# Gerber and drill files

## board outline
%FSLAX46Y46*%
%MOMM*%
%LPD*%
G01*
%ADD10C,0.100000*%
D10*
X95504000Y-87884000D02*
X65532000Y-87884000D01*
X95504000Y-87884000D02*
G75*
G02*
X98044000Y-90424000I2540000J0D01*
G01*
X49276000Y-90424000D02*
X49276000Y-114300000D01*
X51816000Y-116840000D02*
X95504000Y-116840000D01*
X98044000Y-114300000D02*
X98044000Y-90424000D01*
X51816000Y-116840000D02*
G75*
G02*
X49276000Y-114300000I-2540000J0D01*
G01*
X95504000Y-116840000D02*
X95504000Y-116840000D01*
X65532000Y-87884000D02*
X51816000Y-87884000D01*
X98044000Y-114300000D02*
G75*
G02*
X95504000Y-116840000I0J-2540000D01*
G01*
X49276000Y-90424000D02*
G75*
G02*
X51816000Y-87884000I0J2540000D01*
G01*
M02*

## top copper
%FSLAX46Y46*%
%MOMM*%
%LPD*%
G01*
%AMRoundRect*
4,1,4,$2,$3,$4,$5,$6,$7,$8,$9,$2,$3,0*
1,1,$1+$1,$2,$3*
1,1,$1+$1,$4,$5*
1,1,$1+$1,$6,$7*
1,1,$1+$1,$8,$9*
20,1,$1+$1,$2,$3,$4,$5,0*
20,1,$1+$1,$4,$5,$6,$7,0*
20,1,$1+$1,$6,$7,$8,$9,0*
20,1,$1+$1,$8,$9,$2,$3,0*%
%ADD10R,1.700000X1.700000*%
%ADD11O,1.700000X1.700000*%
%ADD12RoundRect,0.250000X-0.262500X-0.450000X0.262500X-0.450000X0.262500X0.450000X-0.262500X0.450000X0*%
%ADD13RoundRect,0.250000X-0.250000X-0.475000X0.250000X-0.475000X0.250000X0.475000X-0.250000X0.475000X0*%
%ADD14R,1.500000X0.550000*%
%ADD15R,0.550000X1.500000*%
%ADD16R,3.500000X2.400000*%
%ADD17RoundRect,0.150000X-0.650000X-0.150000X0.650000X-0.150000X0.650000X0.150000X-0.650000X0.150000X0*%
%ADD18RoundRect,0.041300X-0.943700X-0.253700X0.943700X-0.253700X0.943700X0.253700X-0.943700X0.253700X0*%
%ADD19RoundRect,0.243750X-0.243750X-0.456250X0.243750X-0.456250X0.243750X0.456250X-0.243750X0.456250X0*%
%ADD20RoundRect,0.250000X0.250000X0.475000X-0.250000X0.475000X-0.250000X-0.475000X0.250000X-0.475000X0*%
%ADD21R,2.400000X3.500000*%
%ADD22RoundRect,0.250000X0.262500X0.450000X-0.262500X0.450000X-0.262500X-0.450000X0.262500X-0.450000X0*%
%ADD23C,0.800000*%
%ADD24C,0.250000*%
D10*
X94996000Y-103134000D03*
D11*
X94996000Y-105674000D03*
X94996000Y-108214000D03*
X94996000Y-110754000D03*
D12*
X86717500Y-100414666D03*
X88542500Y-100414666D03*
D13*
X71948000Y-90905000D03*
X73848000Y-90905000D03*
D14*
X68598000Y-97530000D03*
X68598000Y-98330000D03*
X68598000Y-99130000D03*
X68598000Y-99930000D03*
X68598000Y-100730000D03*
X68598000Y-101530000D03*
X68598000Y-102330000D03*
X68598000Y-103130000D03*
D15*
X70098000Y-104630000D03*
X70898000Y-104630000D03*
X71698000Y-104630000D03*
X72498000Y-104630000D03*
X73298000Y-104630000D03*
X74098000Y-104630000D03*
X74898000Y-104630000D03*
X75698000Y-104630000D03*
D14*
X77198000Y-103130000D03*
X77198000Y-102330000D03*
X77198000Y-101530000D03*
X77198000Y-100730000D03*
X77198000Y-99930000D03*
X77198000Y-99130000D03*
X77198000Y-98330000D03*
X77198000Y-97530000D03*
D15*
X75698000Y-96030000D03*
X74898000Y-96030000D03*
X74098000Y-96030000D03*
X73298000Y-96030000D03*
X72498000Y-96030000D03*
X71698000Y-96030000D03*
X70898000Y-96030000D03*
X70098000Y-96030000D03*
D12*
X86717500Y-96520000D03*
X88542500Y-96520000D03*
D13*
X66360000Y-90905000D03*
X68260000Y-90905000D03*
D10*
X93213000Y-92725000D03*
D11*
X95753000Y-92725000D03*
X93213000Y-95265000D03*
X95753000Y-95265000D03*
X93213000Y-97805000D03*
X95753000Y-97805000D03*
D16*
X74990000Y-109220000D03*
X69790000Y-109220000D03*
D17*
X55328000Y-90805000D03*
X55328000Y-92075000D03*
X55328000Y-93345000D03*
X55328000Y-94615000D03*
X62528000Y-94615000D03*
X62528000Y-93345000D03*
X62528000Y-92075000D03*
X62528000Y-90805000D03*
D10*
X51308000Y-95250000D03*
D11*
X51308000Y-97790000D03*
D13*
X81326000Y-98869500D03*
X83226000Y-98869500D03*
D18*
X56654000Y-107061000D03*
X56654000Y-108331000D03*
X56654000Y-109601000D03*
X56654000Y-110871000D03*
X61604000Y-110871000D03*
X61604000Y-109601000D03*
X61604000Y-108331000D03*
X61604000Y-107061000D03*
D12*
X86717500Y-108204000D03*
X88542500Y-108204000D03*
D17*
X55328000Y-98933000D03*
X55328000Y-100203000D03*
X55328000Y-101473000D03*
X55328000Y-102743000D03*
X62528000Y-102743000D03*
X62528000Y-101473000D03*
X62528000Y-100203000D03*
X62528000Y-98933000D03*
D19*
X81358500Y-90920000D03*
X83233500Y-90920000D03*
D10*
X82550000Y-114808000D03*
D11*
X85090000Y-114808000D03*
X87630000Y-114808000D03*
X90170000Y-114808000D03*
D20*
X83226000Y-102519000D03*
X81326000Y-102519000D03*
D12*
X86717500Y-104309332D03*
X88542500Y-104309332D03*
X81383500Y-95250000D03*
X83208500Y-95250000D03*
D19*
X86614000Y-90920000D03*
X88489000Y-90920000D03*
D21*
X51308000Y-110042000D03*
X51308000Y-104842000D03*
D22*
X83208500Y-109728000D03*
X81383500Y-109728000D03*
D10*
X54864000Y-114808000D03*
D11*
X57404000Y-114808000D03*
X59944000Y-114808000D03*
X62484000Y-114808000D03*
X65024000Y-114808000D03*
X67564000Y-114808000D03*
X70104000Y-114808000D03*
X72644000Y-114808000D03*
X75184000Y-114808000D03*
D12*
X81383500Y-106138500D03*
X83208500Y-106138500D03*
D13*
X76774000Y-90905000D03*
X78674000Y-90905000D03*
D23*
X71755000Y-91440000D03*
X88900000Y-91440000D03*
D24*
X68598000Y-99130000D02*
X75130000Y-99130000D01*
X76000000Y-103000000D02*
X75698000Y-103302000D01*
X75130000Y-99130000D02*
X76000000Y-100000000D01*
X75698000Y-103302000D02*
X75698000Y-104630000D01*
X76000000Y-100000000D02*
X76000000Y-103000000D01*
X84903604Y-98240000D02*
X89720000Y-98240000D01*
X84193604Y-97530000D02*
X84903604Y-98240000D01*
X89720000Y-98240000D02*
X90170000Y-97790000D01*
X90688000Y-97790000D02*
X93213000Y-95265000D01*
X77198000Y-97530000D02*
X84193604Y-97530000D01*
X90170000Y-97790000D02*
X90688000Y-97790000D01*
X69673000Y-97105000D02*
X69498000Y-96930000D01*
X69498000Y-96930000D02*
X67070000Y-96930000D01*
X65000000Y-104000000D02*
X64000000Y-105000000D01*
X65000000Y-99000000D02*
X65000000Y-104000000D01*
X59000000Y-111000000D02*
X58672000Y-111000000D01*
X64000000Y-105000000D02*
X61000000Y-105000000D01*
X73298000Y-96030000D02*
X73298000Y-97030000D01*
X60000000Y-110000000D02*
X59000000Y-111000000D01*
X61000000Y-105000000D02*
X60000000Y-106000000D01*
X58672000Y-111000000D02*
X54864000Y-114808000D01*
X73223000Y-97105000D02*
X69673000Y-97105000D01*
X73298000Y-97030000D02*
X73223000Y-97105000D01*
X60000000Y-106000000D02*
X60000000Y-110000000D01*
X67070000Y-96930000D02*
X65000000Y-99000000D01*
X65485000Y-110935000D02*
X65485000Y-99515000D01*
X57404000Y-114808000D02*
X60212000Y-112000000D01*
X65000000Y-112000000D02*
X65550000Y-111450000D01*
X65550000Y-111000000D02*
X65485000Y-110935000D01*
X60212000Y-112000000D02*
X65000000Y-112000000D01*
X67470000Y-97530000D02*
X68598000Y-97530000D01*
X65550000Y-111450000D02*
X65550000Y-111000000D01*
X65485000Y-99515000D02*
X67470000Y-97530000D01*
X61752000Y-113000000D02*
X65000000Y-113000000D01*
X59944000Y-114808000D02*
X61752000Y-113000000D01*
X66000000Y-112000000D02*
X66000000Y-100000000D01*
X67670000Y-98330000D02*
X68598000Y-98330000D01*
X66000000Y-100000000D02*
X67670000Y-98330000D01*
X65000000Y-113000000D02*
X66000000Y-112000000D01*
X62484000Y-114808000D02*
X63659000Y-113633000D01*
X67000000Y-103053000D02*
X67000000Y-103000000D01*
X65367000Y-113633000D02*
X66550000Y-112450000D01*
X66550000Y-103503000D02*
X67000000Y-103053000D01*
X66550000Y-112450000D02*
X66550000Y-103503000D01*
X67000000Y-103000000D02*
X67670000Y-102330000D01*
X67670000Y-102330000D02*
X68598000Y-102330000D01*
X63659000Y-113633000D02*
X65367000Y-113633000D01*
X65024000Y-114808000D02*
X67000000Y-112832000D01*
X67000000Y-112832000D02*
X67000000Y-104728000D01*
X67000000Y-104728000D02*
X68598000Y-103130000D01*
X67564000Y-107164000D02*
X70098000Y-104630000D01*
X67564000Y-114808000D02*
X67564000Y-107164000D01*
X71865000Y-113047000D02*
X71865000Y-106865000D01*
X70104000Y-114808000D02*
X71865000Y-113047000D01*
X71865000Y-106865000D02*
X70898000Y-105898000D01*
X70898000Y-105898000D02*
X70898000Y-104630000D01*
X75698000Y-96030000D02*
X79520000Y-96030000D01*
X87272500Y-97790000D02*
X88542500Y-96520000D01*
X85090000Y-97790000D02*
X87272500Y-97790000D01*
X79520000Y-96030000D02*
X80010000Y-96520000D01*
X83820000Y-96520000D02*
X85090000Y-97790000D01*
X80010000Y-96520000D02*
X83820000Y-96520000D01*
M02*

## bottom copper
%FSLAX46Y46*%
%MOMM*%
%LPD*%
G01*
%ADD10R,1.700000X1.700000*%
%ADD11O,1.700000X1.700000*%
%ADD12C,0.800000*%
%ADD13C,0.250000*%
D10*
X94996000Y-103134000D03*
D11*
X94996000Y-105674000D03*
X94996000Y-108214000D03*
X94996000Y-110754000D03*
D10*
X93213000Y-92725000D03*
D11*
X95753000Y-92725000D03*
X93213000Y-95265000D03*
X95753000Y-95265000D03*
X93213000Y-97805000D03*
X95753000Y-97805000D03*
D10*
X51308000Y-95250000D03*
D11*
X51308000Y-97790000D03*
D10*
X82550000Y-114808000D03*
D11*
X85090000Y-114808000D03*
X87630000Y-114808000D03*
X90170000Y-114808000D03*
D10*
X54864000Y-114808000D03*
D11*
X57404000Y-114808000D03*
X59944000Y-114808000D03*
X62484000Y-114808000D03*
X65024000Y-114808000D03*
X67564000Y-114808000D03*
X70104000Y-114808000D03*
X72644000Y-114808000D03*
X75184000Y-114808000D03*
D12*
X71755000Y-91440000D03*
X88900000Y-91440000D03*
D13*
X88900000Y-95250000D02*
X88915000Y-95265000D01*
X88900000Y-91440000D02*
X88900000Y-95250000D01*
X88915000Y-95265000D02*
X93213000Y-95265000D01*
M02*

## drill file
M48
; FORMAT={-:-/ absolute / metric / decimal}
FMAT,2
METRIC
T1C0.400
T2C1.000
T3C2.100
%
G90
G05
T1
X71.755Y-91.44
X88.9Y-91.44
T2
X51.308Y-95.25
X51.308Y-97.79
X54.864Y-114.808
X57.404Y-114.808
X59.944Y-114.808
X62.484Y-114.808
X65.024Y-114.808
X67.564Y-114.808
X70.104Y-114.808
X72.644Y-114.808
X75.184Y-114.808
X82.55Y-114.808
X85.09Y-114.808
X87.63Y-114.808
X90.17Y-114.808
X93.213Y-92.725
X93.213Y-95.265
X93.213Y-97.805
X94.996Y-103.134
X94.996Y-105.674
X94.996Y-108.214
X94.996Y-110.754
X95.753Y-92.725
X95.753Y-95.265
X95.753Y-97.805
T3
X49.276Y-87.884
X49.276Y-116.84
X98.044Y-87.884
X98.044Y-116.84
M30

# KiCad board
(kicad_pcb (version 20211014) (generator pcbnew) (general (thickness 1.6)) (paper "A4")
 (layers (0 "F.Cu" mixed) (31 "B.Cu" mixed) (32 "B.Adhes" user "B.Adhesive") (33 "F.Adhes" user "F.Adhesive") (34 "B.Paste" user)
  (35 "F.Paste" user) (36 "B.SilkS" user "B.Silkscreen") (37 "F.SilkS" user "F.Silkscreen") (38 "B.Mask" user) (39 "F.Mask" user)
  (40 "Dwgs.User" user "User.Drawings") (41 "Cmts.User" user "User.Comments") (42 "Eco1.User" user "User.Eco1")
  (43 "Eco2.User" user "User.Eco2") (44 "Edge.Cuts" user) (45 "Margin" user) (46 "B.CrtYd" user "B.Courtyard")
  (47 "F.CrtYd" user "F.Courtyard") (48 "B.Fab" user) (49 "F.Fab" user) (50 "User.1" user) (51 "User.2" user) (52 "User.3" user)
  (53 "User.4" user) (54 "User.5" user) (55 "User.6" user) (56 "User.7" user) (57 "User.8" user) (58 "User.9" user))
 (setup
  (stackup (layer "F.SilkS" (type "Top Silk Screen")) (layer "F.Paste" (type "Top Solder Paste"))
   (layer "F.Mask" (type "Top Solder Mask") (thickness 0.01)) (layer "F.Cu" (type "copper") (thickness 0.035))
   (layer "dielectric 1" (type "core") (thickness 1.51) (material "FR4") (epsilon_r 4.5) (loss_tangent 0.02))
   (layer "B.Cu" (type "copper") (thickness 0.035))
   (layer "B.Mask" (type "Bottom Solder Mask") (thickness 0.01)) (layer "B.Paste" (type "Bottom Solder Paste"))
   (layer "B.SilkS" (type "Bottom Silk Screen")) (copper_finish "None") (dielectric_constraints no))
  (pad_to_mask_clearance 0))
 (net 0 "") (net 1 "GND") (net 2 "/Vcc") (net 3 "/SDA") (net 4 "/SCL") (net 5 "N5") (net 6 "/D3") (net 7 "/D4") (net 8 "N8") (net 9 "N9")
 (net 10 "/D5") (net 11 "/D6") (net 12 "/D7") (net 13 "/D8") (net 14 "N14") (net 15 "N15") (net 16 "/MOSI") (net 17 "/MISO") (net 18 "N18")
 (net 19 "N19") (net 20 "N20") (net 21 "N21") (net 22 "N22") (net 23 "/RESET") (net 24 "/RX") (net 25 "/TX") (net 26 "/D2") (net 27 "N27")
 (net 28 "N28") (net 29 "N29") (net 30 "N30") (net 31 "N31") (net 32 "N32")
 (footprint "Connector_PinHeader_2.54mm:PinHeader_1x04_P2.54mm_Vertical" (layer "F.Cu") (at 94.996 103.134)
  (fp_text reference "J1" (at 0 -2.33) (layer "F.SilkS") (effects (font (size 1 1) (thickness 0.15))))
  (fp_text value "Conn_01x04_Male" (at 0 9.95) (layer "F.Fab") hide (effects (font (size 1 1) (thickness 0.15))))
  (pad "1" thru_hole rect (at 0 0) (size 1.7 1.7) (drill 1) (layers *.Cu *.Mask) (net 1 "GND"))
  (pad "2" thru_hole oval (at 0 2.54) (size 1.7 1.7) (drill 1) (layers *.Cu *.Mask) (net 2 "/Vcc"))
  (pad "3" thru_hole oval (at 0 5.08) (size 1.7 1.7) (drill 1) (layers *.Cu *.Mask) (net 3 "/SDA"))
  (pad "4" thru_hole oval (at 0 7.62) (size 1.7 1.7) (drill 1) (layers *.Cu *.Mask) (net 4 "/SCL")))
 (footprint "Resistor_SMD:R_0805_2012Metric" (layer "F.Cu") (at 87.63 100.414666)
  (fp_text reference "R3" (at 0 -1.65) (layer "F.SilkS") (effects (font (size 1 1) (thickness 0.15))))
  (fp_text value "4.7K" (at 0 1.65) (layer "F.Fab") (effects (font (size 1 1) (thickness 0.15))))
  (pad "1" smd roundrect (at -0.9125 0) (size 1.025 1.4) (layers "F.Cu" "F.Paste" "F.Mask") (roundrect_rratio 0.243902) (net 2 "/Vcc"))
  (pad "2" smd roundrect (at 0.9125 0) (size 1.025 1.4) (layers "F.Cu" "F.Paste" "F.Mask") (roundrect_rratio 0.243902) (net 3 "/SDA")))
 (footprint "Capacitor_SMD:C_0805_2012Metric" (layer "F.Cu") (at 72.898 90.905)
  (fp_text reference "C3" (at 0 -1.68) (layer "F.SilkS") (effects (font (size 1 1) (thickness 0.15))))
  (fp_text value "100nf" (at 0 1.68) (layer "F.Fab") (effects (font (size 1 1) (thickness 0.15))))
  (pad "1" smd roundrect (at -0.95 0) (size 1 1.45) (layers "F.Cu" "F.Paste" "F.Mask") (roundrect_rratio 0.25) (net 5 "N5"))
  (pad "2" smd roundrect (at 0.95 0) (size 1 1.45) (layers "F.Cu" "F.Paste" "F.Mask") (roundrect_rratio 0.25) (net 1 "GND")))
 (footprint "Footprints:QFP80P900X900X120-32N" (layer "F.Cu") (at 72.898 100.33)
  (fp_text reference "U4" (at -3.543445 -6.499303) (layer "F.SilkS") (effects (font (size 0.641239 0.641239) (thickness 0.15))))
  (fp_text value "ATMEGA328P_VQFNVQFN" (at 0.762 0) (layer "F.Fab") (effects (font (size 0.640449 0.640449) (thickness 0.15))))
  (pad "1" smd rect locked (at -4.3 -2.8) (size 1.5 0.55) (layers "F.Cu" "F.Paste" "F.Mask") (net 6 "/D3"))
  (pad "2" smd rect locked (at -4.3 -2) (size 1.5 0.55) (layers "F.Cu" "F.Paste" "F.Mask") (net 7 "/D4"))
  (pad "3" smd rect locked (at -4.3 -1.2) (size 1.5 0.55) (layers "F.Cu" "F.Paste" "F.Mask") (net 5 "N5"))
  (pad "4" smd rect locked (at -4.3 -0.4) (size 1.5 0.55) (layers "F.Cu" "F.Paste" "F.Mask") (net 1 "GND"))
  (pad "5" smd rect locked (at -4.3 0.4) (size 1.5 0.55) (layers "F.Cu" "F.Paste" "F.Mask") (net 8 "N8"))
  (pad "6" smd rect locked (at -4.3 1.2) (size 1.5 0.55) (layers "F.Cu" "F.Paste" "F.Mask") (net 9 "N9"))
  (pad "7" smd rect locked (at -4.3 2) (size 1.5 0.55) (layers "F.Cu" "F.Paste" "F.Mask") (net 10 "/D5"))
  (pad "8" smd rect locked (at -4.3 2.8) (size 1.5 0.55) (layers "F.Cu" "F.Paste" "F.Mask") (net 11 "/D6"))
  (pad "9" smd rect locked (at -2.8 4.3) (size 0.55 1.5) (layers "F.Cu" "F.Paste" "F.Mask") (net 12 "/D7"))
  (pad "10" smd rect locked (at -2 4.3) (size 0.55 1.5) (layers "F.Cu" "F.Paste" "F.Mask") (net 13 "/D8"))
  (pad "11" smd rect locked (at -1.2 4.3) (size 0.55 1.5) (layers "F.Cu" "F.Paste" "F.Mask") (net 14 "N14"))
  (pad "12" smd rect locked (at -0.4 4.3) (size 0.55 1.5) (layers "F.Cu" "F.Paste" "F.Mask") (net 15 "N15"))
  (pad "13" smd rect locked (at 0.4 4.3) (size 0.55 1.5) (layers "F.Cu" "F.Paste" "F.Mask") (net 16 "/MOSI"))
  (pad "14" smd rect locked (at 1.2 4.3) (size 0.55 1.5) (layers "F.Cu" "F.Paste" "F.Mask") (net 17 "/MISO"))
  (pad "15" smd rect locked (at 2 4.3) (size 0.55 1.5) (layers "F.Cu" "F.Paste" "F.Mask") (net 4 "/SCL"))
  (pad "16" smd rect locked (at 2.8 4.3) (size 0.55 1.5) (layers "F.Cu" "F.Paste" "F.Mask") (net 5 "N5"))
  (pad "17" smd rect locked (at 4.3 2.8) (size 1.5 0.55) (layers "F.Cu" "F.Paste" "F.Mask") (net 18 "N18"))
  (pad "18" smd rect locked (at 4.3 2) (size 1.5 0.55) (layers "F.Cu" "F.Paste" "F.Mask") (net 1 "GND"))
  (pad "19" smd rect locked (at 4.3 1.2) (size 1.5 0.55) (layers "F.Cu" "F.Paste" "F.Mask") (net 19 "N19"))
  (pad "20" smd rect locked (at 4.3 0.4) (size 1.5 0.55) (layers "F.Cu" "F.Paste" "F.Mask") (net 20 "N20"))
  (pad "21" smd rect locked (at 4.3 -0.4) (size 1.5 0.55) (layers "F.Cu" "F.Paste" "F.Mask") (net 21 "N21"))
  (pad "22" smd rect locked (at 4.3 -1.2) (size 1.5 0.55) (layers "F.Cu" "F.Paste" "F.Mask") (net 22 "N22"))
  (pad "23" smd rect locked (at 4.3 -2) (size 1.5 0.55) (layers "F.Cu" "F.Paste" "F.Mask") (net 3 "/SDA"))
  (pad "24" smd rect locked (at 4.3 -2.8) (size 1.5 0.55) (layers "F.Cu" "F.Paste" "F.Mask") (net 4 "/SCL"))
  (pad "25" smd rect locked (at 2.8 -4.3) (size 0.55 1.5) (layers "F.Cu" "F.Paste" "F.Mask") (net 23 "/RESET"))
  (pad "26" smd rect locked (at 2 -4.3) (size 0.55 1.5) (layers "F.Cu" "F.Paste" "F.Mask") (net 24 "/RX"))
  (pad "27" smd rect locked (at 1.2 -4.3) (size 0.55 1.5) (layers "F.Cu" "F.Paste" "F.Mask") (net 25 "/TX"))
  (pad "28" smd rect locked (at 0.4 -4.3) (size 0.55 1.5) (layers "F.Cu" "F.Paste" "F.Mask") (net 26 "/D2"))
  (pad "29" smd rect locked (at -0.4 -4.3) (size 0.55 1.5) (layers "F.Cu" "F.Paste" "F.Mask"))
  (pad "30" smd rect locked (at -1.2 -4.3) (size 0.55 1.5) (layers "F.Cu" "F.Paste" "F.Mask"))
  (pad "31" smd rect locked (at -2 -4.3) (size 0.55 1.5) (layers "F.Cu" "F.Paste" "F.Mask"))
  (pad "32" smd rect locked (at -2.8 -4.3) (size 0.55 1.5) (layers "F.Cu" "F.Paste" "F.Mask")))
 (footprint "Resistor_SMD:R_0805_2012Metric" (layer "F.Cu") (at 87.63 96.52)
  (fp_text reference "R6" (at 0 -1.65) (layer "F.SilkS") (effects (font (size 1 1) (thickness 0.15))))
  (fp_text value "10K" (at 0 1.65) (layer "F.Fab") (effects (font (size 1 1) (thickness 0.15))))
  (pad "1" smd roundrect (at -0.9125 0) (size 1.025 1.4) (layers "F.Cu" "F.Paste" "F.Mask") (roundrect_rratio 0.243902) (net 2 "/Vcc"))
  (pad "2" smd roundrect (at 0.9125 0) (size 1.025 1.4) (layers "F.Cu" "F.Paste" "F.Mask") (roundrect_rratio 0.243902) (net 23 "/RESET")))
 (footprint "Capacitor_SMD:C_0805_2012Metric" (layer "F.Cu") (at 67.31 90.905)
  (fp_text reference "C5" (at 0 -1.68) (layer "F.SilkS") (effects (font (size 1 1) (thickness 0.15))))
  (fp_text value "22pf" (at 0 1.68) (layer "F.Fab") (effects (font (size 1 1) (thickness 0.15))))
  (pad "1" smd roundrect (at -0.95 0) (size 1 1.45) (layers "F.Cu" "F.Paste" "F.Mask") (roundrect_rratio 0.25) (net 1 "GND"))
  (pad "2" smd roundrect (at 0.95 0) (size 1 1.45) (layers "F.Cu" "F.Paste" "F.Mask") (roundrect_rratio 0.25) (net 8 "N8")))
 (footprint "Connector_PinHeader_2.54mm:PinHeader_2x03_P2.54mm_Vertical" (layer "F.Cu") (at 93.213 92.725)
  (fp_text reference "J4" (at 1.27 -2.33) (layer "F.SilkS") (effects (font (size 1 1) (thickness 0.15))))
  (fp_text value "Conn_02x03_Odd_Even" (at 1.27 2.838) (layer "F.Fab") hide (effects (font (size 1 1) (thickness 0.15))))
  (pad "1" thru_hole rect (at 0 0) (size 1.7 1.7) (drill 1) (layers *.Cu *.Mask) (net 17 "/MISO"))
  (pad "2" thru_hole oval (at 2.54 0) (size 1.7 1.7) (drill 1) (layers *.Cu *.Mask) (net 2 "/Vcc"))
  (pad "3" thru_hole oval (at 0 2.54) (size 1.7 1.7) (drill 1) (layers *.Cu *.Mask) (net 4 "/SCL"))
  (pad "4" thru_hole oval (at 2.54 2.54) (size 1.7 1.7) (drill 1) (layers *.Cu *.Mask) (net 16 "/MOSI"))
  (pad "5" thru_hole oval (at 0 5.08) (size 1.7 1.7) (drill 1) (layers *.Cu *.Mask) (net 23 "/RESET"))
  (pad "6" thru_hole oval (at 2.54 5.08) (size 1.7 1.7) (drill 1) (layers *.Cu *.Mask) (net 1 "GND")))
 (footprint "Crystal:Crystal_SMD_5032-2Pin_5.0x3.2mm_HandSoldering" (layer "F.Cu") (at 72.39 109.22 180)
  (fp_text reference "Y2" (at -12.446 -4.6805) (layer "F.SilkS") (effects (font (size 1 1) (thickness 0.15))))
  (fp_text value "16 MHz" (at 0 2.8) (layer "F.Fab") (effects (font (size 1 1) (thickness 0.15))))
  (pad "1" smd rect (at -2.6 0 180) (size 3.5 2.4) (layers "F.Cu" "F.Paste" "F.Mask") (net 9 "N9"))
  (pad "2" smd rect (at 2.6 0 180) (size 3.5 2.4) (layers "F.Cu" "F.Paste" "F.Mask") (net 8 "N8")))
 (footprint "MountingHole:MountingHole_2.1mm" (layer "F.Cu") (at 49.276 116.84)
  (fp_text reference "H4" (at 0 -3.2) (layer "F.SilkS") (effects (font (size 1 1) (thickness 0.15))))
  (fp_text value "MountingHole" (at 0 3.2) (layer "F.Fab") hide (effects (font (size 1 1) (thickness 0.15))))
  (pad "" np_thru_hole circle (at 0 0) (size 2.1 2.1) (drill 2.1) (layers *.Cu *.Mask)))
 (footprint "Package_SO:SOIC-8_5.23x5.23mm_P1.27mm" (layer "F.Cu") (at 58.928 92.71)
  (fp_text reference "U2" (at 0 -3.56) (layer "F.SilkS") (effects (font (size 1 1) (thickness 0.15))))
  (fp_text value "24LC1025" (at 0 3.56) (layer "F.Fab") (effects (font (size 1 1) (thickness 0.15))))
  (pad "1" smd roundrect (at -3.6 -1.905) (size 1.6 0.6) (layers "F.Cu" "F.Paste" "F.Mask") (roundrect_rratio 0.25) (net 2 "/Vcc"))
  (pad "2" smd roundrect (at -3.6 -0.635) (size 1.6 0.6) (layers "F.Cu" "F.Paste" "F.Mask") (roundrect_rratio 0.25) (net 1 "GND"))
  (pad "3" smd roundrect (at -3.6 0.635) (size 1.6 0.6) (layers "F.Cu" "F.Paste" "F.Mask") (roundrect_rratio 0.25) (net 2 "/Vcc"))
  (pad "4" smd roundrect (at -3.6 1.905) (size 1.6 0.6) (layers "F.Cu" "F.Paste" "F.Mask") (roundrect_rratio 0.25) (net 1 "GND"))
  (pad "5" smd roundrect (at 3.6 1.905) (size 1.6 0.6) (layers "F.Cu" "F.Paste" "F.Mask") (roundrect_rratio 0.25) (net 3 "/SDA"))
  (pad "6" smd roundrect (at 3.6 0.635) (size 1.6 0.6) (layers "F.Cu" "F.Paste" "F.Mask") (roundrect_rratio 0.25) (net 4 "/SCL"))
  (pad "7" smd roundrect (at 3.6 -0.635) (size 1.6 0.6) (layers "F.Cu" "F.Paste" "F.Mask") (roundrect_rratio 0.25) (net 1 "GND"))
  (pad "8" smd roundrect (at 3.6 -1.905) (size 1.6 0.6) (layers "F.Cu" "F.Paste" "F.Mask") (roundrect_rratio 0.25) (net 2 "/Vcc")))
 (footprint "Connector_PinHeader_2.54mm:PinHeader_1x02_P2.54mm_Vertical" (layer "F.Cu") (at 51.308 95.25)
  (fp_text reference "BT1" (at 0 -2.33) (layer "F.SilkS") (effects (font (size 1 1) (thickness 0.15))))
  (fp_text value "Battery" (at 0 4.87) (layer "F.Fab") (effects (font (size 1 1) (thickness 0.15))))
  (pad "1" thru_hole rect (at 0 0) (size 1.7 1.7) (drill 1) (layers *.Cu *.Mask) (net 5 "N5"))
  (pad "2" thru_hole oval (at 0 2.54) (size 1.7 1.7) (drill 1) (layers *.Cu *.Mask) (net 1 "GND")))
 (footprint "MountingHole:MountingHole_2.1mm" (layer "F.Cu") (at 98.044 87.884)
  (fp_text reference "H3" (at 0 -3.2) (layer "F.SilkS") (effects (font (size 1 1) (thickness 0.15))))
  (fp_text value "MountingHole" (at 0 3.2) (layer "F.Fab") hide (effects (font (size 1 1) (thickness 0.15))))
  (pad "" np_thru_hole circle (at 0 0) (size 2.1 2.1) (drill 2.1) (layers *.Cu *.Mask)))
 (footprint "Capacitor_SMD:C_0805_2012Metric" (layer "F.Cu") (at 82.276 98.8695)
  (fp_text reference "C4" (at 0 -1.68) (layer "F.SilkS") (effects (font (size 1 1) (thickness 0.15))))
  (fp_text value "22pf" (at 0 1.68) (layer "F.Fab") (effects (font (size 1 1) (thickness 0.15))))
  (pad "1" smd roundrect (at -0.95 0) (size 1 1.45) (layers "F.Cu" "F.Paste" "F.Mask") (roundrect_rratio 0.25) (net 1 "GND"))
  (pad "2" smd roundrect (at 0.95 0) (size 1 1.45) (layers "F.Cu" "F.Paste" "F.Mask") (roundrect_rratio 0.25) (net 9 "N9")))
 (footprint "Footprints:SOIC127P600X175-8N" (layer "F.Cu") (at 59.129 108.966)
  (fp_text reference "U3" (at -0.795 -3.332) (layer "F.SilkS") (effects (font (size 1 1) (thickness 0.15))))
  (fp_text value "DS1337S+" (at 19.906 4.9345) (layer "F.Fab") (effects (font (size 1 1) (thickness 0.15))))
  (pad "1" smd roundrect locked (at -2.475 -1.905) (size 1.97 0.59) (layers "F.Cu" "F.Paste" "F.Mask") (roundrect_rratio 0.07)
   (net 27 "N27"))
  (pad "2" smd roundrect locked (at -2.475 -0.635) (size 1.97 0.59) (layers "F.Cu" "F.Paste" "F.Mask") (roundrect_rratio 0.07)
   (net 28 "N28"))
  (pad "3" smd roundrect locked (at -2.475 0.635) (size 1.97 0.59) (layers "F.Cu" "F.Paste" "F.Mask") (roundrect_rratio 0.07) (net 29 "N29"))
  (pad "4" smd roundrect locked (at -2.475 1.905) (size 1.97 0.59) (layers "F.Cu" "F.Paste" "F.Mask") (roundrect_rratio 0.07) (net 1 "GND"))
  (pad "5" smd roundrect locked (at 2.475 1.905) (size 1.97 0.59) (layers "F.Cu" "F.Paste" "F.Mask") (roundrect_rratio 0.07) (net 3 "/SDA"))
  (pad "6" smd roundrect locked (at 2.475 0.635) (size 1.97 0.59) (layers "F.Cu" "F.Paste" "F.Mask") (roundrect_rratio 0.07) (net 4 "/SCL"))
  (pad "7" smd roundrect locked (at 2.475 -0.635) (size 1.97 0.59) (layers "F.Cu" "F.Paste" "F.Mask") (roundrect_rratio 0.07) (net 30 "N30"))
  (pad "8" smd roundrect locked (at 2.475 -1.905) (size 1.97 0.59) (layers "F.Cu" "F.Paste" "F.Mask") (roundrect_rratio 0.07) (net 2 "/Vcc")))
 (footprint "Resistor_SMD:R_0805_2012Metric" (layer "F.Cu") (at 87.63 108.204)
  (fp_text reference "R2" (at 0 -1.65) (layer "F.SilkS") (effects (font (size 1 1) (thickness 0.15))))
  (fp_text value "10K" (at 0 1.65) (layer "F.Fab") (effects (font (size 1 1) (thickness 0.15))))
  (pad "1" smd roundrect (at -0.9125 0) (size 1.025 1.4) (layers "F.Cu" "F.Paste" "F.Mask") (roundrect_rratio 0.243902) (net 2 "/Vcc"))
  (pad "2" smd roundrect (at 0.9125 0) (size 1.025 1.4) (layers "F.Cu" "F.Paste" "F.Mask") (roundrect_rratio 0.243902) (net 29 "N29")))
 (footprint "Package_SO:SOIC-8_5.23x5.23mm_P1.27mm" (layer "F.Cu") (at 58.928 100.838)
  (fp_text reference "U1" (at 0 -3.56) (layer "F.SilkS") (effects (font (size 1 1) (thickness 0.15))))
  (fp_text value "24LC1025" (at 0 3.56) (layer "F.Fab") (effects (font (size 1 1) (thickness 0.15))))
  (pad "1" smd roundrect (at -3.6 -1.905) (size 1.6 0.6) (layers "F.Cu" "F.Paste" "F.Mask") (roundrect_rratio 0.25) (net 2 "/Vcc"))
  (pad "2" smd roundrect (at -3.6 -0.635) (size 1.6 0.6) (layers "F.Cu" "F.Paste" "F.Mask") (roundrect_rratio 0.25) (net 2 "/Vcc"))
  (pad "3" smd roundrect (at -3.6 0.635) (size 1.6 0.6) (layers "F.Cu" "F.Paste" "F.Mask") (roundrect_rratio 0.25) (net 2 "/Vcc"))
  (pad "4" smd roundrect (at -3.6 1.905) (size 1.6 0.6) (layers "F.Cu" "F.Paste" "F.Mask") (roundrect_rratio 0.25) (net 1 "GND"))
  (pad "5" smd roundrect (at 3.6 1.905) (size 1.6 0.6) (layers "F.Cu" "F.Paste" "F.Mask") (roundrect_rratio 0.25) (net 3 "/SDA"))
  (pad "6" smd roundrect (at 3.6 0.635) (size 1.6 0.6) (layers "F.Cu" "F.Paste" "F.Mask") (roundrect_rratio 0.25) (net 4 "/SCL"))
  (pad "7" smd roundrect (at 3.6 -0.635) (size 1.6 0.6) (layers "F.Cu" "F.Paste" "F.Mask") (roundrect_rratio 0.25) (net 1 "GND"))
  (pad "8" smd roundrect (at 3.6 -1.905) (size 1.6 0.6) (layers "F.Cu" "F.Paste" "F.Mask") (roundrect_rratio 0.25) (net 2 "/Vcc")))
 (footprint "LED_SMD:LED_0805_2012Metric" (layer "F.Cu") (at 82.296 90.92)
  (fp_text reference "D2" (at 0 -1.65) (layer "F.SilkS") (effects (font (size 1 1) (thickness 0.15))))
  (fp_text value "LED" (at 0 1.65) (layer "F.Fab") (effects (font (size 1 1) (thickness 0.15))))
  (pad "1" smd roundrect (at -0.9375 0) (size 0.975 1.4) (layers "F.Cu" "F.Paste" "F.Mask") (roundrect_rratio 0.25) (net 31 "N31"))
  (pad "2" smd roundrect (at 0.9375 0) (size 0.975 1.4) (layers "F.Cu" "F.Paste" "F.Mask") (roundrect_rratio 0.25) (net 5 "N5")))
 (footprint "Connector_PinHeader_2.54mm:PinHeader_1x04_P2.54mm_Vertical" (layer "F.Cu") (at 82.55 114.808 90)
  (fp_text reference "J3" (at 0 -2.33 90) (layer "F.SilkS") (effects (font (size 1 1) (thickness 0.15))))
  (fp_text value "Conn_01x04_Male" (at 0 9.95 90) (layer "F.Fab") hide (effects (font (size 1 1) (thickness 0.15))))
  (pad "1" thru_hole rect (at 0 0 90) (size 1.7 1.7) (drill 1) (layers *.Cu *.Mask) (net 1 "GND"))
  (pad "2" thru_hole oval (at 0 2.54 90) (size 1.7 1.7) (drill 1) (layers *.Cu *.Mask) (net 2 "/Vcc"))
  (pad "3" thru_hole oval (at 0 5.08 90) (size 1.7 1.7) (drill 1) (layers *.Cu *.Mask) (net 24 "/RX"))
  (pad "4" thru_hole oval (at 0 7.62 90) (size 1.7 1.7) (drill 1) (layers *.Cu *.Mask) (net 25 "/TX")))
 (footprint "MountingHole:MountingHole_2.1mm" (layer "F.Cu") (at 49.276 87.884)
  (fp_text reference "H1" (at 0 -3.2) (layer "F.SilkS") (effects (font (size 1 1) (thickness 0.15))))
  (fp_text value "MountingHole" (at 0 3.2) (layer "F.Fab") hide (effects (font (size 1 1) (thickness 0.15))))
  (pad "" np_thru_hole circle (at 0 0) (size 2.1 2.1) (drill 2.1) (layers *.Cu *.Mask)))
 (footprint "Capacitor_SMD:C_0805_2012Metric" (layer "F.Cu") (at 82.276 102.519 180)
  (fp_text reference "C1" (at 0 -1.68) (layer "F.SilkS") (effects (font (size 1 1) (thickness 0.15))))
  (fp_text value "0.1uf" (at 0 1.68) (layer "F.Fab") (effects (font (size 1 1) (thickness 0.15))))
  (pad "1" smd roundrect (at -0.95 0 180) (size 1 1.45) (layers "F.Cu" "F.Paste" "F.Mask") (roundrect_rratio 0.25) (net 2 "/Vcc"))
  (pad "2" smd roundrect (at 0.95 0 180) (size 1 1.45) (layers "F.Cu" "F.Paste" "F.Mask") (roundrect_rratio 0.25) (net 1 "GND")))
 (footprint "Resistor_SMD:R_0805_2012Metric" (layer "F.Cu") (at 87.63 104.309332)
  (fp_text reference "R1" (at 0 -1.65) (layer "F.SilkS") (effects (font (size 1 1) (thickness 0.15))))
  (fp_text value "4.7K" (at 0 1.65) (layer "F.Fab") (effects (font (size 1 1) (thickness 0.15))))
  (pad "1" smd roundrect (at -0.9125 0) (size 1.025 1.4) (layers "F.Cu" "F.Paste" "F.Mask") (roundrect_rratio 0.243902) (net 2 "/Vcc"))
  (pad "2" smd roundrect (at 0.9125 0) (size 1.025 1.4) (layers "F.Cu" "F.Paste" "F.Mask") (roundrect_rratio 0.243902) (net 4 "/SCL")))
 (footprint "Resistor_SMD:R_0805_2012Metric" (layer "F.Cu") (at 82.296 95.25)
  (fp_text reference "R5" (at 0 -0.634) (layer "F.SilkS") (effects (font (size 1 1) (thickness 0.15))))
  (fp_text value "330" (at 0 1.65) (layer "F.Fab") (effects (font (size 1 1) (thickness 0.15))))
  (pad "1" smd roundrect (at -0.9125 0) (size 1.025 1.4) (layers "F.Cu" "F.Paste" "F.Mask") (roundrect_rratio 0.243902) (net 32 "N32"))
  (pad "2" smd roundrect (at 0.9125 0) (size 1.025 1.4) (layers "F.Cu" "F.Paste" "F.Mask") (roundrect_rratio 0.243902) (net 1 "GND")))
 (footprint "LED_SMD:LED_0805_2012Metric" (layer "F.Cu") (at 87.5515 90.92)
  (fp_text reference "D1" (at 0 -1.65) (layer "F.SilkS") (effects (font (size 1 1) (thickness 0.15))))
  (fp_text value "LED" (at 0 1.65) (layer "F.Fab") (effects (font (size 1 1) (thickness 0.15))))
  (pad "1" smd roundrect (at -0.9375 0) (size 0.975 1.4) (layers "F.Cu" "F.Paste" "F.Mask") (roundrect_rratio 0.25) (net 32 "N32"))
  (pad "2" smd roundrect (at 0.9375 0) (size 0.975 1.4) (layers "F.Cu" "F.Paste" "F.Mask") (roundrect_rratio 0.25) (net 4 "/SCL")))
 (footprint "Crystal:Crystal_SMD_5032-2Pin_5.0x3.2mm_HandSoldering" (layer "F.Cu") (at 51.308 107.442 90)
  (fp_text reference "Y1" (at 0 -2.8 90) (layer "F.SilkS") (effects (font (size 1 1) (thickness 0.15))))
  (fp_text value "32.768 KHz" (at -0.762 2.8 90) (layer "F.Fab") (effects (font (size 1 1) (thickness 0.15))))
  (pad "1" smd rect (at -2.6 0 90) (size 3.5 2.4) (layers "F.Cu" "F.Paste" "F.Mask") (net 28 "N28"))
  (pad "2" smd rect (at 2.6 0 90) (size 3.5 2.4) (layers "F.Cu" "F.Paste" "F.Mask") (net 27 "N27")))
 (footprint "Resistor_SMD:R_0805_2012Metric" (layer "F.Cu") (at 82.296 109.728 180)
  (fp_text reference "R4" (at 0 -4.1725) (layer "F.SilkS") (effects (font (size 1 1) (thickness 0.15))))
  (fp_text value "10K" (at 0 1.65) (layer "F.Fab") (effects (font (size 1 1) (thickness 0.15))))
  (pad "1" smd roundrect (at -0.9125 0 180) (size 1.025 1.4) (layers "F.Cu" "F.Paste" "F.Mask") (roundrect_rratio 0.243902) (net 2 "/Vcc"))
  (pad "2" smd roundrect (at 0.9125 0 180) (size 1.025 1.4) (layers "F.Cu" "F.Paste" "F.Mask") (roundrect_rratio 0.243902) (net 30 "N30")))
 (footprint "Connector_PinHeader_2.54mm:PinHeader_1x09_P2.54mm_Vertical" (layer "F.Cu") (at 54.864 114.808 90)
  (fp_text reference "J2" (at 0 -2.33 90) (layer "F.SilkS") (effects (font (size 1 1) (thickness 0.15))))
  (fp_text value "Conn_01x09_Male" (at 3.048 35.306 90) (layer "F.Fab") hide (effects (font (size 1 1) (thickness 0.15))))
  (pad "1" thru_hole rect (at 0 0 90) (size 1.7 1.7) (drill 1) (layers *.Cu *.Mask) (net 26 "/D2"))
  (pad "2" thru_hole oval (at 0 2.54 90) (size 1.7 1.7) (drill 1) (layers *.Cu *.Mask) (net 6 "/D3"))
  (pad "3" thru_hole oval (at 0 5.08 90) (size 1.7 1.7) (drill 1) (layers *.Cu *.Mask) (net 7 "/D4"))
  (pad "4" thru_hole oval (at 0 7.62 90) (size 1.7 1.7) (drill 1) (layers *.Cu *.Mask) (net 10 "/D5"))
  (pad "5" thru_hole oval (at 0 10.16 90) (size 1.7 1.7) (drill 1) (layers *.Cu *.Mask) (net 11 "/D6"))
  (pad "6" thru_hole oval (at 0 12.7 90) (size 1.7 1.7) (drill 1) (layers *.Cu *.Mask) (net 12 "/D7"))
  (pad "7" thru_hole oval (at 0 15.24 90) (size 1.7 1.7) (drill 1) (layers *.Cu *.Mask) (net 13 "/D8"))
  (pad "8" thru_hole oval (at 0 17.78 90) (size 1.7 1.7) (drill 1) (layers *.Cu *.Mask) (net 1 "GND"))
  (pad "9" thru_hole oval (at 0 20.32 90) (size 1.7 1.7) (drill 1) (layers *.Cu *.Mask) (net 2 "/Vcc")))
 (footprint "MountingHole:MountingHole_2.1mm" (layer "F.Cu") (at 98.044 116.84)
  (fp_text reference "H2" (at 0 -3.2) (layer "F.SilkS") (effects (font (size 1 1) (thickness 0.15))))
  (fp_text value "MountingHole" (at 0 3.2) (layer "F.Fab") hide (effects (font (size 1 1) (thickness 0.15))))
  (pad "" np_thru_hole circle (at 0 0) (size 2.1 2.1) (drill 2.1) (layers *.Cu *.Mask)))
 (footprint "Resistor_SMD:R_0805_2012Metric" (layer "F.Cu") (at 82.296 106.1385)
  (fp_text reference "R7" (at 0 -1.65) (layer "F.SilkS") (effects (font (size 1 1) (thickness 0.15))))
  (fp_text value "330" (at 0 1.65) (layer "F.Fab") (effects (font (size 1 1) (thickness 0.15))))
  (pad "1" smd roundrect (at -0.9125 0) (size 1.025 1.4) (layers "F.Cu" "F.Paste" "F.Mask") (roundrect_rratio 0.243902) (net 1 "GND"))
  (pad "2" smd roundrect (at 0.9125 0) (size 1.025 1.4) (layers "F.Cu" "F.Paste" "F.Mask") (roundrect_rratio 0.243902) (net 31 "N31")))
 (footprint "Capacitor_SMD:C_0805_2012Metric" (layer "F.Cu") (at 77.724 90.905)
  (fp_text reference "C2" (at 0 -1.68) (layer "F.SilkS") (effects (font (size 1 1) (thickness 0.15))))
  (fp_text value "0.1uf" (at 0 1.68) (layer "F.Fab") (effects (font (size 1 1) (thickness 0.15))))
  (pad "1" smd roundrect (at -0.95 0) (size 1 1.45) (layers "F.Cu" "F.Paste" "F.Mask") (roundrect_rratio 0.25) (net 1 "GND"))
  (pad "2" smd roundrect (at 0.95 0) (size 1 1.45) (layers "F.Cu" "F.Paste" "F.Mask") (roundrect_rratio 0.25) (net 18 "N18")))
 (gr_line (start 95.504 87.884) (end 65.532 87.884) (layer "Edge.Cuts") (width 0.1))
 (gr_arc (start 95.504 87.884) (mid 99.840051 86.087949) (end 98.044 90.424) (layer "Edge.Cuts") (width 0.1))
 (gr_line (start 49.276 90.424) (end 49.276 114.3) (layer "Edge.Cuts") (width 0.1))
 (gr_line (start 51.816 116.84) (end 95.504 116.84) (layer "Edge.Cuts") (width 0.1))
 (gr_line (start 98.044 114.3) (end 98.044 90.424) (layer "Edge.Cuts") (width 0.1))
 (gr_arc (start 51.816 116.84) (mid 47.479949 118.636051) (end 49.276 114.3) (layer "Edge.Cuts") (width 0.1))
 (gr_line (start 95.504 116.84) (end 95.504 116.84) (layer "Edge.Cuts") (width 0.1))
 (gr_line (start 65.532 87.884) (end 51.816 87.884) (layer "Edge.Cuts") (width 0.1))
 (gr_arc (start 98.044 114.3) (mid 99.840051 118.636051) (end 95.504 116.84) (layer "Edge.Cuts") (width 0.1))
 (gr_arc (start 49.276 90.424) (mid 47.479949 86.087949) (end 51.816 87.884) (layer "Edge.Cuts") (width 0.1))
 (segment (start 68.598 99.13) (end 75.13 99.13) (width 0.25) (layer "F.Cu") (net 5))
 (segment (start 76 103) (end 75.698 103.302) (width 0.25) (layer "F.Cu") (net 5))
 (segment (start 75.13 99.13) (end 76 100) (width 0.25) (layer "F.Cu") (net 5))
 (segment (start 75.698 103.302) (end 75.698 104.63) (width 0.25) (layer "F.Cu") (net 5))
 (segment (start 76 100) (end 76 103) (width 0.25) (layer "F.Cu") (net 5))
 (via (at 71.755 91.44) (size 0.8) (drill 0.4) (layers "F.Cu" "B.Cu") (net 5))
 (segment (start 84.903604 98.24) (end 89.72 98.24) (width 0.25) (layer "F.Cu") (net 4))
 (segment (start 84.193604 97.53) (end 84.903604 98.24) (width 0.25) (layer "F.Cu") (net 4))
 (segment (start 89.72 98.24) (end 90.17 97.79) (width 0.25) (layer "F.Cu") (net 4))
 (segment (start 90.688 97.79) (end 93.213 95.265) (width 0.25) (layer "F.Cu") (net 4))
 (segment (start 77.198 97.53) (end 84.193604 97.53) (width 0.25) (layer "F.Cu") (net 4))
 (segment (start 90.17 97.79) (end 90.688 97.79) (width 0.25) (layer "F.Cu") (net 4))
 (via (at 88.9 91.44) (size 0.8) (drill 0.4) (layers "F.Cu" "B.Cu") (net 4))
 (segment (start 88.9 95.25) (end 88.915 95.265) (width 0.25) (layer "B.Cu") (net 4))
 (segment (start 88.9 91.44) (end 88.9 95.25) (width 0.25) (layer "B.Cu") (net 4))
 (segment (start 88.915 95.265) (end 93.213 95.265) (width 0.25) (layer "B.Cu") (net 4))
 (segment (start 69.673 97.105) (end 69.498 96.93) (width 0.25) (layer "F.Cu") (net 26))
 (segment (start 69.498 96.93) (end 67.07 96.93) (width 0.25) (layer "F.Cu") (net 26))
 (segment (start 65 104) (end 64 105) (width 0.25) (layer "F.Cu") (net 26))
 (segment (start 65 99) (end 65 104) (width 0.25) (layer "F.Cu") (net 26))
 (segment (start 59 111) (end 58.672 111) (width 0.25) (layer "F.Cu") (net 26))
 (segment (start 64 105) (end 61 105) (width 0.25) (layer "F.Cu") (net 26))
 (segment (start 73.298 96.03) (end 73.298 97.03) (width 0.25) (layer "F.Cu") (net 26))
 (segment (start 60 110) (end 59 111) (width 0.25) (layer "F.Cu") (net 26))
 (segment (start 61 105) (end 60 106) (width 0.25) (layer "F.Cu") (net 26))
 (segment (start 58.672 111) (end 54.864 114.808) (width 0.25) (layer "F.Cu") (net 26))
 (segment (start 73.223 97.105) (end 69.673 97.105) (width 0.25) (layer "F.Cu") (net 26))
 (segment (start 73.298 97.03) (end 73.223 97.105) (width 0.25) (layer "F.Cu") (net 26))
 (segment (start 60 106) (end 60 110) (width 0.25) (layer "F.Cu") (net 26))
 (segment (start 67.07 96.93) (end 65 99) (width 0.25) (layer "F.Cu") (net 26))
 (segment (start 65.485 110.935) (end 65.485 99.515) (width 0.25) (layer "F.Cu") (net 6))
 (segment (start 57.404 114.808) (end 60.212 112) (width 0.25) (layer "F.Cu") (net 6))
 (segment (start 65 112) (end 65.55 111.45) (width 0.25) (layer "F.Cu") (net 6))
 (segment (start 65.55 111) (end 65.485 110.935) (width 0.25) (layer "F.Cu") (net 6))
 (segment (start 60.212 112) (end 65 112) (width 0.25) (layer "F.Cu") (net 6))
 (segment (start 67.47 97.53) (end 68.598 97.53) (width 0.25) (layer "F.Cu") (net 6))
 (segment (start 65.55 111.45) (end 65.55 111) (width 0.25) (layer "F.Cu") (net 6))
 (segment (start 65.485 99.515) (end 67.47 97.53) (width 0.25) (layer "F.Cu") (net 6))
 (segment (start 61.752 113) (end 65 113) (width 0.25) (layer "F.Cu") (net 7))
 (segment (start 59.944 114.808) (end 61.752 113) (width 0.25) (layer "F.Cu") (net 7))
 (segment (start 66 112) (end 66 100) (width 0.25) (layer "F.Cu") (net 7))
 (segment (start 67.67 98.33) (end 68.598 98.33) (width 0.25) (layer "F.Cu") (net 7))
 (segment (start 66 100) (end 67.67 98.33) (width 0.25) (layer "F.Cu") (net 7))
 (segment (start 65 113) (end 66 112) (width 0.25) (layer "F.Cu") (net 7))
 (segment (start 62.484 114.808) (end 63.659 113.633) (width 0.25) (layer "F.Cu") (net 10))
 (segment (start 67 103.053) (end 67 103) (width 0.25) (layer "F.Cu") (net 10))
 (segment (start 65.367 113.633) (end 66.55 112.45) (width 0.25) (layer "F.Cu") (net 10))
 (segment (start 66.55 103.503) (end 67 103.053) (width 0.25) (layer "F.Cu") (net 10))
 (segment (start 66.55 112.45) (end 66.55 103.503) (width 0.25) (layer "F.Cu") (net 10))
 (segment (start 67 103) (end 67.67 102.33) (width 0.25) (layer "F.Cu") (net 10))
 (segment (start 67.67 102.33) (end 68.598 102.33) (width 0.25) (layer "F.Cu") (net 10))
 (segment (start 63.659 113.633) (end 65.367 113.633) (width 0.25) (layer "F.Cu") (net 10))
 (segment (start 65.024 114.808) (end 67 112.832) (width 0.25) (layer "F.Cu") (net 11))
 (segment (start 67 112.832) (end 67 104.728) (width 0.25) (layer "F.Cu") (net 11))
 (segment (start 67 104.728) (end 68.598 103.13) (width 0.25) (layer "F.Cu") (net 11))
 (segment (start 67.564 107.164) (end 70.098 104.63) (width 0.25) (layer "F.Cu") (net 12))
 (segment (start 67.564 114.808) (end 67.564 107.164) (width 0.25) (layer "F.Cu") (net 12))
 (segment (start 71.865 113.047) (end 71.865 106.865) (width 0.25) (layer "F.Cu") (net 13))
 (segment (start 70.104 114.808) (end 71.865 113.047) (width 0.25) (layer "F.Cu") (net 13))
 (segment (start 71.865 106.865) (end 70.898 105.898) (width 0.25) (layer "F.Cu") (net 13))
 (segment (start 70.898 105.898) (end 70.898 104.63) (width 0.25) (layer "F.Cu") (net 13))
 (segment (start 75.698 96.03) (end 79.52 96.03) (width 0.25) (layer "F.Cu") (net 23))
 (segment (start 87.2725 97.79) (end 88.5425 96.52) (width 0.25) (layer "F.Cu") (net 23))
 (segment (start 85.09 97.79) (end 87.2725 97.79) (width 0.25) (layer "F.Cu") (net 23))
 (segment (start 79.52 96.03) (end 80.01 96.52) (width 0.25) (layer "F.Cu") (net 23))
 (segment (start 83.82 96.52) (end 85.09 97.79) (width 0.25) (layer "F.Cu") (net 23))
 (segment (start 80.01 96.52) (end 83.82 96.52) (width 0.25) (layer "F.Cu") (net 23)))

